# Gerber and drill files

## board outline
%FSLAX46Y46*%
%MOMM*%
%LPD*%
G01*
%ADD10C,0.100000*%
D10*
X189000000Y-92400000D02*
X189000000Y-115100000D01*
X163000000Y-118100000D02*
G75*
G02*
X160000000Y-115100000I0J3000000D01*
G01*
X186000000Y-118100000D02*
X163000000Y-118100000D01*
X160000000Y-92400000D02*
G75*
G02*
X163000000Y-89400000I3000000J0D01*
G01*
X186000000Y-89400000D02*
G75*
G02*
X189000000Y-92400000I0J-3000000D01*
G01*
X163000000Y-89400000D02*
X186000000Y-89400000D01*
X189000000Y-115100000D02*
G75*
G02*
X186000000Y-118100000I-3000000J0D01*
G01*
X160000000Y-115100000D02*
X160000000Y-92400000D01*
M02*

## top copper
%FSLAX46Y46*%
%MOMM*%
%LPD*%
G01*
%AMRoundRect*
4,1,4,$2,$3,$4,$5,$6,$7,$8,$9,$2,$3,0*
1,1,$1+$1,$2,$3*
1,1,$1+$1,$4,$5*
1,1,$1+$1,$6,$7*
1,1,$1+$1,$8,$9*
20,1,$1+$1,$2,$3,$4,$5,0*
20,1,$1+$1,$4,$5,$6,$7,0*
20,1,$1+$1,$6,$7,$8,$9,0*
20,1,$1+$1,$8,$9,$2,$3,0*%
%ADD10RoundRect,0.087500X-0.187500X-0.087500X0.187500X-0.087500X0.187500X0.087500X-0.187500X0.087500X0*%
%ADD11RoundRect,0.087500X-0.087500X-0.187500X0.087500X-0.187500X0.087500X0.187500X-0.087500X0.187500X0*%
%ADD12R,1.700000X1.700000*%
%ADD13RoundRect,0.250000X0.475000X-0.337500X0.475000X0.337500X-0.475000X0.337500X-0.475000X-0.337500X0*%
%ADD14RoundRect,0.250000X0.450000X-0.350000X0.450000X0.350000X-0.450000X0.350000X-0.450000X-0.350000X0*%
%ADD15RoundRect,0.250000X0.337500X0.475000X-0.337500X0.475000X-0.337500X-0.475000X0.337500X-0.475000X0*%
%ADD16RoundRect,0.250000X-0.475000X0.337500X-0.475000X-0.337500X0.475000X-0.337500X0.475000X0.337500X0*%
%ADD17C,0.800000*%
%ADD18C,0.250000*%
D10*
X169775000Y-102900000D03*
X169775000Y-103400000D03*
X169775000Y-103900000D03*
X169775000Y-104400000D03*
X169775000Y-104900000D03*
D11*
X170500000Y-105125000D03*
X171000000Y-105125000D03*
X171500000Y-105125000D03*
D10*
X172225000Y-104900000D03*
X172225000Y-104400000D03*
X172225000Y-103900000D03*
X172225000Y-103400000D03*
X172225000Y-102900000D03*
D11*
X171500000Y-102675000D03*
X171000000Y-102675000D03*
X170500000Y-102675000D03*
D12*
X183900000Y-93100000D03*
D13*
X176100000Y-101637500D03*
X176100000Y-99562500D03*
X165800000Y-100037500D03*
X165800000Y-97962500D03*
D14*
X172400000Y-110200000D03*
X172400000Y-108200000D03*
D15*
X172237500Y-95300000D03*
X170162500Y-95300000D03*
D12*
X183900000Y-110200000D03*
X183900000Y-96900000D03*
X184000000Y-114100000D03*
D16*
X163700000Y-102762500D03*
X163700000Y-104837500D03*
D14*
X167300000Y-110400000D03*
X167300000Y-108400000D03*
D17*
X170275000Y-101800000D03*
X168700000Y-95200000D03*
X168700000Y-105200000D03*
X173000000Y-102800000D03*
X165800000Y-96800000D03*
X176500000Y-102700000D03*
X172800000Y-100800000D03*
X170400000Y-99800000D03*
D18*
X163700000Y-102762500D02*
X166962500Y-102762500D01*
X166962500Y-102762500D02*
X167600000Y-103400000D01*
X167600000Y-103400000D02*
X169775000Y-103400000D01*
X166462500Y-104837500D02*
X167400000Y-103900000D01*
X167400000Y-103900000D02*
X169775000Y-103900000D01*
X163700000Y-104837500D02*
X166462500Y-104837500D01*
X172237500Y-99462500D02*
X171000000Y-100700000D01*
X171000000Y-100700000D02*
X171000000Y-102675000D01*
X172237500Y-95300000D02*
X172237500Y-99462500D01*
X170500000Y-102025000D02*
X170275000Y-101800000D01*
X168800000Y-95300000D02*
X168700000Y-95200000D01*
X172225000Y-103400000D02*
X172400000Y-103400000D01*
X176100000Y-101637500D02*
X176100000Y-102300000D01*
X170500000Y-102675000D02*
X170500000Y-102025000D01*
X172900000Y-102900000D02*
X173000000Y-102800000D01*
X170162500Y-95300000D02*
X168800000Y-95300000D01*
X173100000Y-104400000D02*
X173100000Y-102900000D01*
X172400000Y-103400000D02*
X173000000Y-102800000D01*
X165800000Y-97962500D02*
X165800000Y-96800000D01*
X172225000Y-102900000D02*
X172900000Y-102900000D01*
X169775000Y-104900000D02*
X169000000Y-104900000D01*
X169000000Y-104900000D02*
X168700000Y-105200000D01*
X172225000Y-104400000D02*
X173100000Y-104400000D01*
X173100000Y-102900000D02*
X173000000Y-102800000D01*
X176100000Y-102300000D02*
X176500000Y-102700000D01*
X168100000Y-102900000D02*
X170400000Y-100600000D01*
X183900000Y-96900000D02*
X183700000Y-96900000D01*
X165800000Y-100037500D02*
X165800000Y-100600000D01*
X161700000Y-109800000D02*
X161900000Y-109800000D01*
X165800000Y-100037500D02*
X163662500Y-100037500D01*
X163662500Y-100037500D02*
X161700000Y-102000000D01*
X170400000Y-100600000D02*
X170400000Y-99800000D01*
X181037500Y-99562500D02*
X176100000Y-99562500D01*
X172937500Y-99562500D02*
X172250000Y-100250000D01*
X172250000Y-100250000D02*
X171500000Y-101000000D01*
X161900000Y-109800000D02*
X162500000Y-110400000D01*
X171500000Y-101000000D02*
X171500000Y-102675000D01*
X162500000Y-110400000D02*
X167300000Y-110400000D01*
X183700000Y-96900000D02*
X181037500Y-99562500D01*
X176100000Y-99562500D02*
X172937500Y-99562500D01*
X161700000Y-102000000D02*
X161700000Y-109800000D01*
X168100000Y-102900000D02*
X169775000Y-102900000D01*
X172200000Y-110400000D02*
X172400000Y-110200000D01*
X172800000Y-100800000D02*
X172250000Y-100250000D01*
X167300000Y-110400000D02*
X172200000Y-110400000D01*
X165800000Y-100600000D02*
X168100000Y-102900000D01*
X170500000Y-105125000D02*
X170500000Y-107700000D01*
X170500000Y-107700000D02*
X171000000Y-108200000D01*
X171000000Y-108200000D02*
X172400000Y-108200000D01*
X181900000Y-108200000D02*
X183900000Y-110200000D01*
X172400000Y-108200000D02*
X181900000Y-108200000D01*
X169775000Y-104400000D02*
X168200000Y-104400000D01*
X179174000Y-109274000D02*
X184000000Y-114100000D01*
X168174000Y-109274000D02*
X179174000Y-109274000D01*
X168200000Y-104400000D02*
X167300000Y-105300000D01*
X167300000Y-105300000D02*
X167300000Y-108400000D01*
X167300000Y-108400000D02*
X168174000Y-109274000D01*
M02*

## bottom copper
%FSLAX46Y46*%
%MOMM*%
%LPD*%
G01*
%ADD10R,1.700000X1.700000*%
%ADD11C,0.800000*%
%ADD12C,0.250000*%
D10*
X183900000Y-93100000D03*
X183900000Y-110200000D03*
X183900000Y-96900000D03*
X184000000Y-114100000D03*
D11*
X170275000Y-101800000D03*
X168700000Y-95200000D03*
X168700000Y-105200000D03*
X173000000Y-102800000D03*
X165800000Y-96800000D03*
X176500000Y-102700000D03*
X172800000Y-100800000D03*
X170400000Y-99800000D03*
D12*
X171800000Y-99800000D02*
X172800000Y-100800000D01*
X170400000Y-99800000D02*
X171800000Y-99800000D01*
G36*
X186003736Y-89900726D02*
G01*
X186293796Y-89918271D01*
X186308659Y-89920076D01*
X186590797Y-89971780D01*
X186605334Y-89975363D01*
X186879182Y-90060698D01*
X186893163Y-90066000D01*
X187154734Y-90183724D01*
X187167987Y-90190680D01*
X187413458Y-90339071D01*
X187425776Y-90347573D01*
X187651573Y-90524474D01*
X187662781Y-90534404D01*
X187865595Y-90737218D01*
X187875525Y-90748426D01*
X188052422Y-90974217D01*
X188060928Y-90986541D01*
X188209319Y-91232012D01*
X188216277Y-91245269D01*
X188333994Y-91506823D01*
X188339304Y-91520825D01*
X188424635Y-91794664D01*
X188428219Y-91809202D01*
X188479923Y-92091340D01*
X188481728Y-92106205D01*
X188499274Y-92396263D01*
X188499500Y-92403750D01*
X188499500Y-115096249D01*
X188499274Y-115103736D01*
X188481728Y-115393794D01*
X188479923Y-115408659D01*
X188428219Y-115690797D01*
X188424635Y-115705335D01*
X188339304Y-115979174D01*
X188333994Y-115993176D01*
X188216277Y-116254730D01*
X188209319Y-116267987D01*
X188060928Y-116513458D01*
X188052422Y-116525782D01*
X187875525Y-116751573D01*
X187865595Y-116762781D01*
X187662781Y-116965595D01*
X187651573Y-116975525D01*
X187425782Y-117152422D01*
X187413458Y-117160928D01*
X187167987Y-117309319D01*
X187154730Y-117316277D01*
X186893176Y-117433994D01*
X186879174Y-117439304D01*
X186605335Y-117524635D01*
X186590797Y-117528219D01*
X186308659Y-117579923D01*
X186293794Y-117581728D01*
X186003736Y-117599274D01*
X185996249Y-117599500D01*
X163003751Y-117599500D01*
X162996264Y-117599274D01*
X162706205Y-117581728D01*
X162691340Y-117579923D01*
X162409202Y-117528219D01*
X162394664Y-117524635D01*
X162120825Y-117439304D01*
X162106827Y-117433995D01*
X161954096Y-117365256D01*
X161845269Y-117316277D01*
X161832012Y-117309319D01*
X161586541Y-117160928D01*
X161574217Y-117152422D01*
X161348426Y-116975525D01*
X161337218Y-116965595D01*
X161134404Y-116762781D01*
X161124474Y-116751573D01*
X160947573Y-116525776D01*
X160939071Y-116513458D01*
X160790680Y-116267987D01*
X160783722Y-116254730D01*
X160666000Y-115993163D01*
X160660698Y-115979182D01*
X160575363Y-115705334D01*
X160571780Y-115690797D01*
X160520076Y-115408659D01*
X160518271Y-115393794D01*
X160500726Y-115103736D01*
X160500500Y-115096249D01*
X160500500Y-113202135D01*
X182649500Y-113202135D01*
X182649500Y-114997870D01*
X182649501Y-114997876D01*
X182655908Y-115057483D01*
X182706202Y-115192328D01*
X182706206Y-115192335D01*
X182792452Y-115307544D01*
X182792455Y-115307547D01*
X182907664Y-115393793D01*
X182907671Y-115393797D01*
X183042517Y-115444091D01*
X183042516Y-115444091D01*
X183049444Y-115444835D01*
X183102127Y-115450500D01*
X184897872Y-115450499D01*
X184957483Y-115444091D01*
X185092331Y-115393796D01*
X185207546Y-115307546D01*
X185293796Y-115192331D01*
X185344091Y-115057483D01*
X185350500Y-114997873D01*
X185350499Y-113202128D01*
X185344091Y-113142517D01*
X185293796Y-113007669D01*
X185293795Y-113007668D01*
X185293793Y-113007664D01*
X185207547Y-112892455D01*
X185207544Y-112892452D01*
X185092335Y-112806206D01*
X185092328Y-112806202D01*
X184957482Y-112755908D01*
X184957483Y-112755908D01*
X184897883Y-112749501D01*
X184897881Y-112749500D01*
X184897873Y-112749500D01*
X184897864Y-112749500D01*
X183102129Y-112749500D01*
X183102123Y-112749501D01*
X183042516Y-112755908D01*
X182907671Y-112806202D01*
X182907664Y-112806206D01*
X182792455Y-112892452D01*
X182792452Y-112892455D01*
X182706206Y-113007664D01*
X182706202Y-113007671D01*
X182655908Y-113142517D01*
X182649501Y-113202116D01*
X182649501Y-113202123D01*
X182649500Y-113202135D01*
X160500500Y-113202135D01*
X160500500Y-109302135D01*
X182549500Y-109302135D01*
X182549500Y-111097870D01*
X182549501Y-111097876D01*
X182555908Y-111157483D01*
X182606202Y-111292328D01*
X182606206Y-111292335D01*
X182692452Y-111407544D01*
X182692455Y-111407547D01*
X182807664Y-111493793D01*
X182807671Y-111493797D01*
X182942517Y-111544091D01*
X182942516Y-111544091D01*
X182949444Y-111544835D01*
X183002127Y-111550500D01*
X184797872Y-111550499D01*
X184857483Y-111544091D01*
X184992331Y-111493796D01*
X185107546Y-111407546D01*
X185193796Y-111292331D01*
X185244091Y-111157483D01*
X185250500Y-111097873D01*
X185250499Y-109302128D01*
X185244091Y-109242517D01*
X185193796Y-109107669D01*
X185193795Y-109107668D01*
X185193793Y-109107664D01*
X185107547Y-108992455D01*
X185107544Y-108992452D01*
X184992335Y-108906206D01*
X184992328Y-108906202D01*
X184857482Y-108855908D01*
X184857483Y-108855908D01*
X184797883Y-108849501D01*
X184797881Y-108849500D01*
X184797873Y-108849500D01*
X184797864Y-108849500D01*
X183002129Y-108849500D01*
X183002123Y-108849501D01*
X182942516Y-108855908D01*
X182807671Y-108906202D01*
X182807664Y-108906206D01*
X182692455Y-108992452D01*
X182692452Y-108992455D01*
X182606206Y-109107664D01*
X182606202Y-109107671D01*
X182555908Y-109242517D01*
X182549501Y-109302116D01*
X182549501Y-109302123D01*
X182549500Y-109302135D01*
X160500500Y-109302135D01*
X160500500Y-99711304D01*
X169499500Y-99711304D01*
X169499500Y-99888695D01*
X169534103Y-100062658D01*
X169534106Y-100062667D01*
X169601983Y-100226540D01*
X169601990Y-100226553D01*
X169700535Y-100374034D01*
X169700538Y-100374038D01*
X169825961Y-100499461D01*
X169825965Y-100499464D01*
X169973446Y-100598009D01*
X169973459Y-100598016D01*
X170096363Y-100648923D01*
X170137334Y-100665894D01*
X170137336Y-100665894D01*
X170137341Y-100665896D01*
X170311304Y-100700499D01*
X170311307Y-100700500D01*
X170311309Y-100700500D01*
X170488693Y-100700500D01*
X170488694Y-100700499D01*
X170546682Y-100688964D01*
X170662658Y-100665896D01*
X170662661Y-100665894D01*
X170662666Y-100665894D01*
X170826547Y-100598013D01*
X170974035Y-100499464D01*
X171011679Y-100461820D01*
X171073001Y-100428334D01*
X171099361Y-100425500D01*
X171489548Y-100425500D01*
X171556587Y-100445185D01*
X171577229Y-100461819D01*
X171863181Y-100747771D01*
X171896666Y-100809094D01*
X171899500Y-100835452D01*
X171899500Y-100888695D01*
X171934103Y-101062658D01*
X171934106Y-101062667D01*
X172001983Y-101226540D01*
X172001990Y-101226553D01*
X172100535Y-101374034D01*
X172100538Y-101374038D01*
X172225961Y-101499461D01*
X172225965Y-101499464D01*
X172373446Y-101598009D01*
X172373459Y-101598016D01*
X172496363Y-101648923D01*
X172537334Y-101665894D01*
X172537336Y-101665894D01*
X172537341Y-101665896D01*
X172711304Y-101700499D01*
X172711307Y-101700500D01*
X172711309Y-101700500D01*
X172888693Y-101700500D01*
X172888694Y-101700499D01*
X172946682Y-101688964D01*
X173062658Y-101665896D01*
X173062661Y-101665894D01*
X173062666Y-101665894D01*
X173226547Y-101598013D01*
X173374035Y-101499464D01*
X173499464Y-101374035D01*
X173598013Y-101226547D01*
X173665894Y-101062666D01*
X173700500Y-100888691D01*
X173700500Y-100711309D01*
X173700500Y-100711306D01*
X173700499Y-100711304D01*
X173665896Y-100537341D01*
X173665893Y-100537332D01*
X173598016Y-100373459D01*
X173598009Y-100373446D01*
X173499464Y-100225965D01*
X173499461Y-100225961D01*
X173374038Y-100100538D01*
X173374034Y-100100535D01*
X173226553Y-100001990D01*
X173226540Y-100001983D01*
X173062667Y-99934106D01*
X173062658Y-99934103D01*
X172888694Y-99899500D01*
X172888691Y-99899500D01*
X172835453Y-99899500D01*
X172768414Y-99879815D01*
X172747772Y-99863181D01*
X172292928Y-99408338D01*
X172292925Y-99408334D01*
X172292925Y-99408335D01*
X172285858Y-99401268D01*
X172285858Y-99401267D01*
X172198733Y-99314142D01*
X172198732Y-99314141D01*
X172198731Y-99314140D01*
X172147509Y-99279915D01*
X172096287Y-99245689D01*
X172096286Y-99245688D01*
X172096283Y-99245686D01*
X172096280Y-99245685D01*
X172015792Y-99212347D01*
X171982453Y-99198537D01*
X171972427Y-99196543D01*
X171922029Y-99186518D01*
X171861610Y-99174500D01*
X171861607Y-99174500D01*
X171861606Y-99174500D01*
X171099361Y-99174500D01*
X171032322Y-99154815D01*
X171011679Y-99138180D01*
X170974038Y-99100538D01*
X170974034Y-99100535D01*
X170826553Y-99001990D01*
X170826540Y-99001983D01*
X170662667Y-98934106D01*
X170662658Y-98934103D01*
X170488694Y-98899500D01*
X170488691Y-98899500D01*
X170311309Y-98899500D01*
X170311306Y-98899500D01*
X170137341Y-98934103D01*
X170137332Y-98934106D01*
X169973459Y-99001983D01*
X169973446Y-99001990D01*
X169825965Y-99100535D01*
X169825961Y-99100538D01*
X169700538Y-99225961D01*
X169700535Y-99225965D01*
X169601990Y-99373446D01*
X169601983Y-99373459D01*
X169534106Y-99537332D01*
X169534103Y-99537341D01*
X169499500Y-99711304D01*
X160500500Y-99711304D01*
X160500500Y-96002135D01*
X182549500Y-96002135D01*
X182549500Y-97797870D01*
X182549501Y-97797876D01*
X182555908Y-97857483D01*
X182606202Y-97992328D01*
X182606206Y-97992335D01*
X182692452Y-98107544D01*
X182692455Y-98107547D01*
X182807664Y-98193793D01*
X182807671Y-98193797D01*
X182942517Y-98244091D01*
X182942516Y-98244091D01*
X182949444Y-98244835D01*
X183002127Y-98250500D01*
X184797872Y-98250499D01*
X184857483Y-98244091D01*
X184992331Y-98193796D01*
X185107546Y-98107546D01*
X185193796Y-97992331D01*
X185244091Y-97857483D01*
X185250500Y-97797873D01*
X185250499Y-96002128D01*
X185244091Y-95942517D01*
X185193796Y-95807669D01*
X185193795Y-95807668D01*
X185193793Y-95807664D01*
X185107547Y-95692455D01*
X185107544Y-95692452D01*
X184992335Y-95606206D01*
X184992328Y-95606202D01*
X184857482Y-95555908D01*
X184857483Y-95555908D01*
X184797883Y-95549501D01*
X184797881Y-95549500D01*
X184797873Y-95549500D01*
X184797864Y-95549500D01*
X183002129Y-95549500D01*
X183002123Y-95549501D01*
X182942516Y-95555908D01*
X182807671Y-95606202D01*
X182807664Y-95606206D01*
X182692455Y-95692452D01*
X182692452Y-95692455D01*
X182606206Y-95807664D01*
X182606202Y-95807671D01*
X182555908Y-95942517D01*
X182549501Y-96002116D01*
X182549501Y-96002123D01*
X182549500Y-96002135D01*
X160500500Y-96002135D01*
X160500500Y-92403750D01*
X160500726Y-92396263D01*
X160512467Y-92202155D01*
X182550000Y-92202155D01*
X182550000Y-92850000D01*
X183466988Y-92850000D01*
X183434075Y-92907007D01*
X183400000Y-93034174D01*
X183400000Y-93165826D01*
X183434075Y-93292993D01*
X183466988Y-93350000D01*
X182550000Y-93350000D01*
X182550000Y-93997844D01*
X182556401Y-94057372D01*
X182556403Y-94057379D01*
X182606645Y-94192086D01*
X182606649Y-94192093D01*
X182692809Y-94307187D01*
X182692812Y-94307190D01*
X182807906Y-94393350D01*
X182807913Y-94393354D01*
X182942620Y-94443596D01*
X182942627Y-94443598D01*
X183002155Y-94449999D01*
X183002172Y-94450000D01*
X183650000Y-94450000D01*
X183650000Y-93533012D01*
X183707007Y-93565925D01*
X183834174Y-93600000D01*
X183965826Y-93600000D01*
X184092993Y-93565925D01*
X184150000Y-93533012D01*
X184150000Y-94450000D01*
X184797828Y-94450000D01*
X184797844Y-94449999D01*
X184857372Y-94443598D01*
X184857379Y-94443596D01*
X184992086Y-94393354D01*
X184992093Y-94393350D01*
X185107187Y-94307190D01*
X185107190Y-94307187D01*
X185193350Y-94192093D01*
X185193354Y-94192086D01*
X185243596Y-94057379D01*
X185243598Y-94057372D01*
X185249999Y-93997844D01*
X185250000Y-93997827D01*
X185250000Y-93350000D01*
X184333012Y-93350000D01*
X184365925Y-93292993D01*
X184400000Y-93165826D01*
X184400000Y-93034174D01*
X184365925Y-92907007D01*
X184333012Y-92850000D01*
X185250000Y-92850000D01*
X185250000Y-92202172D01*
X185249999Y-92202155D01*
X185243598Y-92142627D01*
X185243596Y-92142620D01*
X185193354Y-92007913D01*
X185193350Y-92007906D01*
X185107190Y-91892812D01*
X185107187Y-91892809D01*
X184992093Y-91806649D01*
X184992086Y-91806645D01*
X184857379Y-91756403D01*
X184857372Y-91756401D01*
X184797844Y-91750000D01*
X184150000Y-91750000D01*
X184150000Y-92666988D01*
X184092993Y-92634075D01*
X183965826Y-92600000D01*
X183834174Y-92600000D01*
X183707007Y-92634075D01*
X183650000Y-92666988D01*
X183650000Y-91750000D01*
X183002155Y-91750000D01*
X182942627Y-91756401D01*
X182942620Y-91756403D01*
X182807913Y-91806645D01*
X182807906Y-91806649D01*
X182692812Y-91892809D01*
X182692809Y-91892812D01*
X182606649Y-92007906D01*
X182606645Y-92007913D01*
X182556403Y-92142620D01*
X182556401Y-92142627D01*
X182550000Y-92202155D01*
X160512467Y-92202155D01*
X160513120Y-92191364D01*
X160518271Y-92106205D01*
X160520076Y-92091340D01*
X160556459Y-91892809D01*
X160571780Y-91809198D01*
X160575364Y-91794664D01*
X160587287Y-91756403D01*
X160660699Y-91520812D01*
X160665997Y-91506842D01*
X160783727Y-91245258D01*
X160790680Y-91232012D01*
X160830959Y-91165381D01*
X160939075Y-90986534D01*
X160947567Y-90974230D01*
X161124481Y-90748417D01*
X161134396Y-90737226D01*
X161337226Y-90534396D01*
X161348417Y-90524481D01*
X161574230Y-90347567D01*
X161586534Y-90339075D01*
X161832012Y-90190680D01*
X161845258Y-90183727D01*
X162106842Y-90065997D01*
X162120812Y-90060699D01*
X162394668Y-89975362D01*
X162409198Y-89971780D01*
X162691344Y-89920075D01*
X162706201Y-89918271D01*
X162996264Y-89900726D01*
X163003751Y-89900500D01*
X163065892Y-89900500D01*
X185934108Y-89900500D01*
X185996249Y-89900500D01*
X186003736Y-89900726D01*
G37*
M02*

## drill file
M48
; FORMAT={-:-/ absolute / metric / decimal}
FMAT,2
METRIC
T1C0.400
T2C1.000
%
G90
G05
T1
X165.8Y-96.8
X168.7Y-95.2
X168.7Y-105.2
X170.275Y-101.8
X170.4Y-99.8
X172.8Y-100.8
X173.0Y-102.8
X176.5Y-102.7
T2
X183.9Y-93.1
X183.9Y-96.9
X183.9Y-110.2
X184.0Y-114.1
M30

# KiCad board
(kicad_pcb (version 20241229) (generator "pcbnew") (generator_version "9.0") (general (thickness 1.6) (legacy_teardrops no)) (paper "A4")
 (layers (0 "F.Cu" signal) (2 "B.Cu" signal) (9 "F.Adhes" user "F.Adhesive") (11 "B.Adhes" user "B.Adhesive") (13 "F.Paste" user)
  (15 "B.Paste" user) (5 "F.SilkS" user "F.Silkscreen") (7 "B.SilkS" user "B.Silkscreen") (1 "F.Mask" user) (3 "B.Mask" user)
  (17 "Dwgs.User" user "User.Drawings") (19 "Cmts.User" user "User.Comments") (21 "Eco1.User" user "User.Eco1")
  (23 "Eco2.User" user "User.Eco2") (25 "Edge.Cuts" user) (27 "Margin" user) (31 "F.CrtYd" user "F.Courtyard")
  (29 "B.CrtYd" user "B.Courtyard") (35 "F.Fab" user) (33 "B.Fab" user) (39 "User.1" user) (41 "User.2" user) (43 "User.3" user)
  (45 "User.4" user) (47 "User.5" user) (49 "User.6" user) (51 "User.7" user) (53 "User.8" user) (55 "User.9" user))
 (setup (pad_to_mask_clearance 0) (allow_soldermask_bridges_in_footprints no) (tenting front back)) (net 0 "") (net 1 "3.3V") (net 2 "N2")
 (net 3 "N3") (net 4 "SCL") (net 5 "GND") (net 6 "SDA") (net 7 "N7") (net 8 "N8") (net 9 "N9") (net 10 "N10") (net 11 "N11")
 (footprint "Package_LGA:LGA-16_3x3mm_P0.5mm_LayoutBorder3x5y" (layer "F.Cu") (at 171 103.9)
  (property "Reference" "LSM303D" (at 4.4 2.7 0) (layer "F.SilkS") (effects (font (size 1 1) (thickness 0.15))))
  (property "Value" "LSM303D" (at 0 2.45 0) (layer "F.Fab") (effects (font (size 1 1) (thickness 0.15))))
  (pad "1" smd roundrect (at -1.225 -1) (size 0.55 0.35) (layers "F.Cu" "F.Mask" "F.Paste") (roundrect_rratio 0.25) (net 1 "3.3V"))
  (pad "2" smd roundrect (at -1.225 -0.5) (size 0.55 0.35) (layers "F.Cu" "F.Mask" "F.Paste") (roundrect_rratio 0.25) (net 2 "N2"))
  (pad "3" smd roundrect (at -1.225 0) (size 0.55 0.35) (layers "F.Cu" "F.Mask" "F.Paste") (roundrect_rratio 0.25) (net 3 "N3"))
  (pad "4" smd roundrect (at -1.225 0.5) (size 0.55 0.35) (layers "F.Cu" "F.Mask" "F.Paste") (roundrect_rratio 0.25) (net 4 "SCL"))
  (pad "5" smd roundrect (at -1.225 1) (size 0.55 0.35) (layers "F.Cu" "F.Mask" "F.Paste") (roundrect_rratio 0.25) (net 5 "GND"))
  (pad "6" smd roundrect (at -0.5 1.225) (size 0.35 0.55) (layers "F.Cu" "F.Mask" "F.Paste") (roundrect_rratio 0.25) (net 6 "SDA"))
  (pad "7" smd roundrect (at 0 1.225) (size 0.35 0.55) (layers "F.Cu" "F.Mask" "F.Paste") (roundrect_rratio 0.25) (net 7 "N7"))
  (pad "8" smd roundrect (at 0.5 1.225) (size 0.35 0.55) (layers "F.Cu" "F.Mask" "F.Paste") (roundrect_rratio 0.25) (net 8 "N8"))
  (pad "9" smd roundrect (at 1.225 1) (size 0.55 0.35) (layers "F.Cu" "F.Mask" "F.Paste") (roundrect_rratio 0.25) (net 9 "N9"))
  (pad "10" smd roundrect (at 1.225 0.5) (size 0.55 0.35) (layers "F.Cu" "F.Mask" "F.Paste") (roundrect_rratio 0.25) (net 5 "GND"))
  (pad "11" smd roundrect (at 1.225 0) (size 0.55 0.35) (layers "F.Cu" "F.Mask" "F.Paste") (roundrect_rratio 0.25) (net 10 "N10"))
  (pad "12" smd roundrect (at 1.225 -0.5) (size 0.55 0.35) (layers "F.Cu" "F.Mask" "F.Paste") (roundrect_rratio 0.25) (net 5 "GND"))
  (pad "13" smd roundrect (at 1.225 -1) (size 0.55 0.35) (layers "F.Cu" "F.Mask" "F.Paste") (roundrect_rratio 0.25) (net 5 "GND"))
  (pad "14" smd roundrect (at 0.5 -1.225) (size 0.35 0.55) (layers "F.Cu" "F.Mask" "F.Paste") (roundrect_rratio 0.25) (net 1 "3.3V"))
  (pad "15" smd roundrect (at 0 -1.225) (size 0.35 0.55) (layers "F.Cu" "F.Mask" "F.Paste") (roundrect_rratio 0.25) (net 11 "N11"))
  (pad "16" smd roundrect (at -0.5 -1.225) (size 0.35 0.55) (layers "F.Cu" "F.Mask" "F.Paste") (roundrect_rratio 0.25) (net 5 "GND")))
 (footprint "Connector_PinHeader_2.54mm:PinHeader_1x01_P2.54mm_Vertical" (layer "F.Cu") (at 183.9 93.1)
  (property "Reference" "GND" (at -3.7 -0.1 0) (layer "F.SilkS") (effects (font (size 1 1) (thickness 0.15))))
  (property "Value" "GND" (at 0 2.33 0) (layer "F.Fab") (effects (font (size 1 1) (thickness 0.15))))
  (pad "1" thru_hole rect (at 0 0) (size 1.7 1.7) (drill 1) (layers "*.Cu" "*.Mask") (remove_unused_layers no) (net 5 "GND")))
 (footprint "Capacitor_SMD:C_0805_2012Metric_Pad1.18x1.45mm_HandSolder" (layer "F.Cu") (at 176.1 100.6 90)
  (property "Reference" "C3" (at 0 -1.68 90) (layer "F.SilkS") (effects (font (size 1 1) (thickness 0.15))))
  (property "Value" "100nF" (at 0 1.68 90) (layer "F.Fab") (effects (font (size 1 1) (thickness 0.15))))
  (pad "1" smd roundrect (at -1.0375 0 90) (size 1.175 1.45) (layers "F.Cu" "F.Mask" "F.Paste") (roundrect_rratio 0.212766) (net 5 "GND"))
  (pad "2" smd roundrect (at 1.0375 0 90) (size 1.175 1.45) (layers "F.Cu" "F.Mask" "F.Paste") (roundrect_rratio 0.212766) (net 1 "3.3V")))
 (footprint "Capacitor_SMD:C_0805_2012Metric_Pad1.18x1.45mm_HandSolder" (layer "F.Cu") (at 165.8 99 90)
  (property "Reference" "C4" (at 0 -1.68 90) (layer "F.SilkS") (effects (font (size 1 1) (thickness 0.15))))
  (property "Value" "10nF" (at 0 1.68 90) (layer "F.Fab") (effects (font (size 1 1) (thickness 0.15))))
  (pad "1" smd roundrect (at -1.0375 0 90) (size 1.175 1.45) (layers "F.Cu" "F.Mask" "F.Paste") (roundrect_rratio 0.212766) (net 1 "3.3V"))
  (pad "2" smd roundrect (at 1.0375 0 90) (size 1.175 1.45) (layers "F.Cu" "F.Mask" "F.Paste") (roundrect_rratio 0.212766) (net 5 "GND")))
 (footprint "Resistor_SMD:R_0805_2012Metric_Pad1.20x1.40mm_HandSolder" (layer "F.Cu") (at 172.4 109.2 90)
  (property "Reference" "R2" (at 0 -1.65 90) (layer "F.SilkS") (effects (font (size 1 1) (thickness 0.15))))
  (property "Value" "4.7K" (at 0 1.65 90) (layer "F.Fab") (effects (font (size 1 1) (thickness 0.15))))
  (pad "1" smd roundrect (at -1 0 90) (size 1.2 1.4) (layers "F.Cu" "F.Mask" "F.Paste") (roundrect_rratio 0.208333) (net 1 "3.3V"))
  (pad "2" smd roundrect (at 1 0 90) (size 1.2 1.4) (layers "F.Cu" "F.Mask" "F.Paste") (roundrect_rratio 0.208333) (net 6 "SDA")))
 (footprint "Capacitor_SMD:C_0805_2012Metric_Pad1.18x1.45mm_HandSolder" (layer "F.Cu") (at 171.2 95.3 180)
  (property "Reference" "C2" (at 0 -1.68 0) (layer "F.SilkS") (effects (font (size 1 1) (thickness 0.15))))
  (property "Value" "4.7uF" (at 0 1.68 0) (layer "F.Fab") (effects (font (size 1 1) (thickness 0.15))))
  (pad "1" smd roundrect (at -1.0375 0 180) (size 1.175 1.45) (layers "F.Cu" "F.Mask" "F.Paste") (roundrect_rratio 0.212766) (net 11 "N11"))
  (pad "2" smd roundrect (at 1.0375 0 180) (size 1.175 1.45) (layers "F.Cu" "F.Mask" "F.Paste") (roundrect_rratio 0.212766) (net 5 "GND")))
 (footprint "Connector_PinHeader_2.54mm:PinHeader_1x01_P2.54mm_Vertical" (layer "F.Cu") (at 183.9 110.2)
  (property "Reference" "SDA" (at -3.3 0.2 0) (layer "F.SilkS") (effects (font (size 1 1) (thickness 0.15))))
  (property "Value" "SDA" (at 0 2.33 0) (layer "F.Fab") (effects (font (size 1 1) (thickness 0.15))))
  (pad "1" thru_hole rect (at 0 0) (size 1.7 1.7) (drill 1) (layers "*.Cu" "*.Mask") (remove_unused_layers no) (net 6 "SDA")))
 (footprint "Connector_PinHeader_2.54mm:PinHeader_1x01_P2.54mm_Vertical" (layer "F.Cu") (at 183.9 96.9)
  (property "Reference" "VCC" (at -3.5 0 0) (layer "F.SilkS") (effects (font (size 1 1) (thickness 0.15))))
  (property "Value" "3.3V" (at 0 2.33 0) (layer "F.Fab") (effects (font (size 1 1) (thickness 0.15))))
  (pad "1" thru_hole rect (at 0 0) (size 1.7 1.7) (drill 1) (layers "*.Cu" "*.Mask") (remove_unused_layers no) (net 1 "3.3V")))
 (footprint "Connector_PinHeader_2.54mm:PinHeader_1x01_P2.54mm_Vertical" (layer "F.Cu") (at 184 114.1)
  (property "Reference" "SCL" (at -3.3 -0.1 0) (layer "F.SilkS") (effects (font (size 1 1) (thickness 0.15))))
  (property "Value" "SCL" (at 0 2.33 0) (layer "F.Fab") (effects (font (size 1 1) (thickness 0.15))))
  (pad "1" thru_hole rect (at 0 0) (size 1.7 1.7) (drill 1) (layers "*.Cu" "*.Mask") (remove_unused_layers no) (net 4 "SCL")))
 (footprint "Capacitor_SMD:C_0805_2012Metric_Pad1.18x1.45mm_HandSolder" (layer "F.Cu") (at 163.7 103.8 -90)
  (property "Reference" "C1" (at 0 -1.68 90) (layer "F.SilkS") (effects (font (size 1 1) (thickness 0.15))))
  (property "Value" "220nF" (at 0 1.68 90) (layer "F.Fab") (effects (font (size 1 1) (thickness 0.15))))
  (pad "1" smd roundrect (at -1.0375 0 270) (size 1.175 1.45) (layers "F.Cu" "F.Mask" "F.Paste") (roundrect_rratio 0.212766) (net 2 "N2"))
  (pad "2" smd roundrect (at 1.0375 0 270) (size 1.175 1.45) (layers "F.Cu" "F.Mask" "F.Paste") (roundrect_rratio 0.212766) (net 3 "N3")))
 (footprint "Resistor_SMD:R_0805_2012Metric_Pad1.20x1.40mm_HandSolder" (layer "F.Cu") (at 167.3 109.4 90)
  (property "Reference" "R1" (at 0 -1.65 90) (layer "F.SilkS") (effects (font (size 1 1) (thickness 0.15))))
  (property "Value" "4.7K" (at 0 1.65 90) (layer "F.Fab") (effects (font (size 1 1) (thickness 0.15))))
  (pad "1" smd roundrect (at -1 0 90) (size 1.2 1.4) (layers "F.Cu" "F.Mask" "F.Paste") (roundrect_rratio 0.208333) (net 1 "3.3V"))
  (pad "2" smd roundrect (at 1 0 90) (size 1.2 1.4) (layers "F.Cu" "F.Mask" "F.Paste") (roundrect_rratio 0.208333) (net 4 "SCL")))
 (gr_line (start 189 92.4) (end 189 115.1) (stroke (width 0.1) (type default)) (layer "Edge.Cuts"))
 (gr_arc (start 163 118.1) (mid 160.87868 117.22132) (end 160 115.1) (stroke (width 0.1) (type default)) (layer "Edge.Cuts"))
 (gr_line (start 186 118.1) (end 163 118.1) (stroke (width 0.1) (type default)) (layer "Edge.Cuts"))
 (gr_arc (start 160 92.4) (mid 160.87868 90.27868) (end 163 89.4) (stroke (width 0.1) (type default)) (layer "Edge.Cuts"))
 (gr_arc (start 186 89.4) (mid 188.12132 90.27868) (end 189 92.4) (stroke (width 0.1) (type default)) (layer "Edge.Cuts"))
 (gr_line (start 163 89.4) (end 186 89.4) (stroke (width 0.1) (type default)) (layer "Edge.Cuts"))
 (gr_arc (start 189 115.1) (mid 188.12132 117.22132) (end 186 118.1) (stroke (width 0.1) (type default)) (layer "Edge.Cuts"))
 (gr_line (start 160 115.1) (end 160 92.4) (stroke (width 0.1) (type default)) (layer "Edge.Cuts"))
 (segment (start 163.7 102.7625) (end 166.9625 102.7625) (width 0.25) (layer "F.Cu") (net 2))
 (segment (start 166.9625 102.7625) (end 167.6 103.4) (width 0.25) (layer "F.Cu") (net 2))
 (segment (start 167.6 103.4) (end 169.775 103.4) (width 0.25) (layer "F.Cu") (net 2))
 (segment (start 166.4625 104.8375) (end 167.4 103.9) (width 0.25) (layer "F.Cu") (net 3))
 (segment (start 167.4 103.9) (end 169.775 103.9) (width 0.25) (layer "F.Cu") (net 3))
 (segment (start 163.7 104.8375) (end 166.4625 104.8375) (width 0.25) (layer "F.Cu") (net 3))
 (segment (start 172.2375 99.4625) (end 171 100.7) (width 0.25) (layer "F.Cu") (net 11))
 (segment (start 171 100.7) (end 171 102.675) (width 0.25) (layer "F.Cu") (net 11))
 (segment (start 172.2375 95.3) (end 172.2375 99.4625) (width 0.25) (layer "F.Cu") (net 11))
 (segment (start 170.5 102.025) (end 170.275 101.8) (width 0.25) (layer "F.Cu") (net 5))
 (segment (start 168.8 95.3) (end 168.7 95.2) (width 0.25) (layer "F.Cu") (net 5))
 (segment (start 172.225 103.4) (end 172.4 103.4) (width 0.25) (layer "F.Cu") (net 5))
 (segment (start 176.1 101.6375) (end 176.1 102.3) (width 0.25) (layer "F.Cu") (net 5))
 (segment (start 170.5 102.675) (end 170.5 102.025) (width 0.25) (layer "F.Cu") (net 5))
 (segment (start 172.9 102.9) (end 173 102.8) (width 0.25) (layer "F.Cu") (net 5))
 (segment (start 170.1625 95.3) (end 168.8 95.3) (width 0.25) (layer "F.Cu") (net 5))
 (segment (start 173.1 104.4) (end 173.1 102.9) (width 0.25) (layer "F.Cu") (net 5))
 (segment (start 172.4 103.4) (end 173 102.8) (width 0.25) (layer "F.Cu") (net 5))
 (segment (start 165.8 97.9625) (end 165.8 96.8) (width 0.25) (layer "F.Cu") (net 5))
 (segment (start 172.225 102.9) (end 172.9 102.9) (width 0.25) (layer "F.Cu") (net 5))
 (segment (start 169.775 104.9) (end 169 104.9) (width 0.25) (layer "F.Cu") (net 5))
 (segment (start 169 104.9) (end 168.7 105.2) (width 0.25) (layer "F.Cu") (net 5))
 (segment (start 172.225 104.4) (end 173.1 104.4) (width 0.25) (layer "F.Cu") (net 5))
 (segment (start 173.1 102.9) (end 173 102.8) (width 0.25) (layer "F.Cu") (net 5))
 (segment (start 176.1 102.3) (end 176.5 102.7) (width 0.25) (layer "F.Cu") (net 5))
 (via (at 170.275 101.8) (size 0.8) (drill 0.4) (layers "F.Cu" "B.Cu") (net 5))
 (via (at 168.7 95.2) (size 0.8) (drill 0.4) (layers "F.Cu" "B.Cu") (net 5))
 (via (at 168.7 105.2) (size 0.8) (drill 0.4) (layers "F.Cu" "B.Cu") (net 5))
 (via (at 173 102.8) (size 0.8) (drill 0.4) (layers "F.Cu" "B.Cu") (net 5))
 (via (at 165.8 96.8) (size 0.8) (drill 0.4) (layers "F.Cu" "B.Cu") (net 5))
 (via (at 176.5 102.7) (size 0.8) (drill 0.4) (layers "F.Cu" "B.Cu") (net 5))
 (segment (start 168.1 102.9) (end 170.4 100.6) (width 0.25) (layer "F.Cu") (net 1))
 (segment (start 183.9 96.9) (end 183.7 96.9) (width 0.25) (layer "F.Cu") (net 1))
 (segment (start 165.8 100.0375) (end 165.8 100.6) (width 0.25) (layer "F.Cu") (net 1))
 (segment (start 161.7 109.8) (end 161.9 109.8) (width 0.25) (layer "F.Cu") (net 1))
 (segment (start 165.8 100.0375) (end 163.6625 100.0375) (width 0.25) (layer "F.Cu") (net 1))
 (segment (start 163.6625 100.0375) (end 161.7 102) (width 0.25) (layer "F.Cu") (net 1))
 (segment (start 170.4 100.6) (end 170.4 99.8) (width 0.25) (layer "F.Cu") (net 1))
 (segment (start 181.0375 99.5625) (end 176.1 99.5625) (width 0.25) (layer "F.Cu") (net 1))
 (segment (start 172.9375 99.5625) (end 172.25 100.25) (width 0.25) (layer "F.Cu") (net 1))
 (segment (start 172.25 100.25) (end 171.5 101) (width 0.25) (layer "F.Cu") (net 1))
 (segment (start 161.9 109.8) (end 162.5 110.4) (width 0.25) (layer "F.Cu") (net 1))
 (segment (start 171.5 101) (end 171.5 102.675) (width 0.25) (layer "F.Cu") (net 1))
 (segment (start 162.5 110.4) (end 167.3 110.4) (width 0.25) (layer "F.Cu") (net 1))
 (segment (start 183.7 96.9) (end 181.0375 99.5625) (width 0.25) (layer "F.Cu") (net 1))
 (segment (start 176.1 99.5625) (end 172.9375 99.5625) (width 0.25) (layer "F.Cu") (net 1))
 (segment (start 161.7 102) (end 161.7 109.8) (width 0.25) (layer "F.Cu") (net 1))
 (segment (start 168.1 102.9) (end 169.775 102.9) (width 0.25) (layer "F.Cu") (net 1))
 (segment (start 172.2 110.4) (end 172.4 110.2) (width 0.25) (layer "F.Cu") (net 1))
 (segment (start 172.8 100.8) (end 172.25 100.25) (width 0.25) (layer "F.Cu") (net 1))
 (segment (start 167.3 110.4) (end 172.2 110.4) (width 0.25) (layer "F.Cu") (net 1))
 (segment (start 165.8 100.6) (end 168.1 102.9) (width 0.25) (layer "F.Cu") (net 1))
 (via (at 172.8 100.8) (size 0.8) (drill 0.4) (layers "F.Cu" "B.Cu") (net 1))
 (via (at 170.4 99.8) (size 0.8) (drill 0.4) (layers "F.Cu" "B.Cu") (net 1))
 (segment (start 171.8 99.8) (end 172.8 100.8) (width 0.25) (layer "B.Cu") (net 1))
 (segment (start 170.4 99.8) (end 171.8 99.8) (width 0.25) (layer "B.Cu") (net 1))
 (segment (start 170.5 105.125) (end 170.5 107.7) (width 0.25) (layer "F.Cu") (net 6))
 (segment (start 170.5 107.7) (end 171 108.2) (width 0.25) (layer "F.Cu") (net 6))
 (segment (start 171 108.2) (end 172.4 108.2) (width 0.25) (layer "F.Cu") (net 6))
 (segment (start 181.9 108.2) (end 183.9 110.2) (width 0.25) (layer "F.Cu") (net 6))
 (segment (start 172.4 108.2) (end 181.9 108.2) (width 0.25) (layer "F.Cu") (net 6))
 (segment (start 169.775 104.4) (end 168.2 104.4) (width 0.25) (layer "F.Cu") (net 4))
 (segment (start 179.174 109.274) (end 184 114.1) (width 0.25) (layer "F.Cu") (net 4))
 (segment (start 168.174 109.274) (end 179.174 109.274) (width 0.25) (layer "F.Cu") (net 4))
 (segment (start 168.2 104.4) (end 167.3 105.3) (width 0.25) (layer "F.Cu") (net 4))
 (segment (start 167.3 105.3) (end 167.3 108.4) (width 0.25) (layer "F.Cu") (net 4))
 (segment (start 167.3 108.4) (end 168.174 109.274) (width 0.25) (layer "F.Cu") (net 4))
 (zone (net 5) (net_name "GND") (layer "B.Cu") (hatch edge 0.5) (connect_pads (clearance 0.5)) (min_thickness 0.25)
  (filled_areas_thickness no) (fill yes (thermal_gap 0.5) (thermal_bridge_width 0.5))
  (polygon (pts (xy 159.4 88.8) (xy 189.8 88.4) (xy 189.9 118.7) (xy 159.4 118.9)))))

